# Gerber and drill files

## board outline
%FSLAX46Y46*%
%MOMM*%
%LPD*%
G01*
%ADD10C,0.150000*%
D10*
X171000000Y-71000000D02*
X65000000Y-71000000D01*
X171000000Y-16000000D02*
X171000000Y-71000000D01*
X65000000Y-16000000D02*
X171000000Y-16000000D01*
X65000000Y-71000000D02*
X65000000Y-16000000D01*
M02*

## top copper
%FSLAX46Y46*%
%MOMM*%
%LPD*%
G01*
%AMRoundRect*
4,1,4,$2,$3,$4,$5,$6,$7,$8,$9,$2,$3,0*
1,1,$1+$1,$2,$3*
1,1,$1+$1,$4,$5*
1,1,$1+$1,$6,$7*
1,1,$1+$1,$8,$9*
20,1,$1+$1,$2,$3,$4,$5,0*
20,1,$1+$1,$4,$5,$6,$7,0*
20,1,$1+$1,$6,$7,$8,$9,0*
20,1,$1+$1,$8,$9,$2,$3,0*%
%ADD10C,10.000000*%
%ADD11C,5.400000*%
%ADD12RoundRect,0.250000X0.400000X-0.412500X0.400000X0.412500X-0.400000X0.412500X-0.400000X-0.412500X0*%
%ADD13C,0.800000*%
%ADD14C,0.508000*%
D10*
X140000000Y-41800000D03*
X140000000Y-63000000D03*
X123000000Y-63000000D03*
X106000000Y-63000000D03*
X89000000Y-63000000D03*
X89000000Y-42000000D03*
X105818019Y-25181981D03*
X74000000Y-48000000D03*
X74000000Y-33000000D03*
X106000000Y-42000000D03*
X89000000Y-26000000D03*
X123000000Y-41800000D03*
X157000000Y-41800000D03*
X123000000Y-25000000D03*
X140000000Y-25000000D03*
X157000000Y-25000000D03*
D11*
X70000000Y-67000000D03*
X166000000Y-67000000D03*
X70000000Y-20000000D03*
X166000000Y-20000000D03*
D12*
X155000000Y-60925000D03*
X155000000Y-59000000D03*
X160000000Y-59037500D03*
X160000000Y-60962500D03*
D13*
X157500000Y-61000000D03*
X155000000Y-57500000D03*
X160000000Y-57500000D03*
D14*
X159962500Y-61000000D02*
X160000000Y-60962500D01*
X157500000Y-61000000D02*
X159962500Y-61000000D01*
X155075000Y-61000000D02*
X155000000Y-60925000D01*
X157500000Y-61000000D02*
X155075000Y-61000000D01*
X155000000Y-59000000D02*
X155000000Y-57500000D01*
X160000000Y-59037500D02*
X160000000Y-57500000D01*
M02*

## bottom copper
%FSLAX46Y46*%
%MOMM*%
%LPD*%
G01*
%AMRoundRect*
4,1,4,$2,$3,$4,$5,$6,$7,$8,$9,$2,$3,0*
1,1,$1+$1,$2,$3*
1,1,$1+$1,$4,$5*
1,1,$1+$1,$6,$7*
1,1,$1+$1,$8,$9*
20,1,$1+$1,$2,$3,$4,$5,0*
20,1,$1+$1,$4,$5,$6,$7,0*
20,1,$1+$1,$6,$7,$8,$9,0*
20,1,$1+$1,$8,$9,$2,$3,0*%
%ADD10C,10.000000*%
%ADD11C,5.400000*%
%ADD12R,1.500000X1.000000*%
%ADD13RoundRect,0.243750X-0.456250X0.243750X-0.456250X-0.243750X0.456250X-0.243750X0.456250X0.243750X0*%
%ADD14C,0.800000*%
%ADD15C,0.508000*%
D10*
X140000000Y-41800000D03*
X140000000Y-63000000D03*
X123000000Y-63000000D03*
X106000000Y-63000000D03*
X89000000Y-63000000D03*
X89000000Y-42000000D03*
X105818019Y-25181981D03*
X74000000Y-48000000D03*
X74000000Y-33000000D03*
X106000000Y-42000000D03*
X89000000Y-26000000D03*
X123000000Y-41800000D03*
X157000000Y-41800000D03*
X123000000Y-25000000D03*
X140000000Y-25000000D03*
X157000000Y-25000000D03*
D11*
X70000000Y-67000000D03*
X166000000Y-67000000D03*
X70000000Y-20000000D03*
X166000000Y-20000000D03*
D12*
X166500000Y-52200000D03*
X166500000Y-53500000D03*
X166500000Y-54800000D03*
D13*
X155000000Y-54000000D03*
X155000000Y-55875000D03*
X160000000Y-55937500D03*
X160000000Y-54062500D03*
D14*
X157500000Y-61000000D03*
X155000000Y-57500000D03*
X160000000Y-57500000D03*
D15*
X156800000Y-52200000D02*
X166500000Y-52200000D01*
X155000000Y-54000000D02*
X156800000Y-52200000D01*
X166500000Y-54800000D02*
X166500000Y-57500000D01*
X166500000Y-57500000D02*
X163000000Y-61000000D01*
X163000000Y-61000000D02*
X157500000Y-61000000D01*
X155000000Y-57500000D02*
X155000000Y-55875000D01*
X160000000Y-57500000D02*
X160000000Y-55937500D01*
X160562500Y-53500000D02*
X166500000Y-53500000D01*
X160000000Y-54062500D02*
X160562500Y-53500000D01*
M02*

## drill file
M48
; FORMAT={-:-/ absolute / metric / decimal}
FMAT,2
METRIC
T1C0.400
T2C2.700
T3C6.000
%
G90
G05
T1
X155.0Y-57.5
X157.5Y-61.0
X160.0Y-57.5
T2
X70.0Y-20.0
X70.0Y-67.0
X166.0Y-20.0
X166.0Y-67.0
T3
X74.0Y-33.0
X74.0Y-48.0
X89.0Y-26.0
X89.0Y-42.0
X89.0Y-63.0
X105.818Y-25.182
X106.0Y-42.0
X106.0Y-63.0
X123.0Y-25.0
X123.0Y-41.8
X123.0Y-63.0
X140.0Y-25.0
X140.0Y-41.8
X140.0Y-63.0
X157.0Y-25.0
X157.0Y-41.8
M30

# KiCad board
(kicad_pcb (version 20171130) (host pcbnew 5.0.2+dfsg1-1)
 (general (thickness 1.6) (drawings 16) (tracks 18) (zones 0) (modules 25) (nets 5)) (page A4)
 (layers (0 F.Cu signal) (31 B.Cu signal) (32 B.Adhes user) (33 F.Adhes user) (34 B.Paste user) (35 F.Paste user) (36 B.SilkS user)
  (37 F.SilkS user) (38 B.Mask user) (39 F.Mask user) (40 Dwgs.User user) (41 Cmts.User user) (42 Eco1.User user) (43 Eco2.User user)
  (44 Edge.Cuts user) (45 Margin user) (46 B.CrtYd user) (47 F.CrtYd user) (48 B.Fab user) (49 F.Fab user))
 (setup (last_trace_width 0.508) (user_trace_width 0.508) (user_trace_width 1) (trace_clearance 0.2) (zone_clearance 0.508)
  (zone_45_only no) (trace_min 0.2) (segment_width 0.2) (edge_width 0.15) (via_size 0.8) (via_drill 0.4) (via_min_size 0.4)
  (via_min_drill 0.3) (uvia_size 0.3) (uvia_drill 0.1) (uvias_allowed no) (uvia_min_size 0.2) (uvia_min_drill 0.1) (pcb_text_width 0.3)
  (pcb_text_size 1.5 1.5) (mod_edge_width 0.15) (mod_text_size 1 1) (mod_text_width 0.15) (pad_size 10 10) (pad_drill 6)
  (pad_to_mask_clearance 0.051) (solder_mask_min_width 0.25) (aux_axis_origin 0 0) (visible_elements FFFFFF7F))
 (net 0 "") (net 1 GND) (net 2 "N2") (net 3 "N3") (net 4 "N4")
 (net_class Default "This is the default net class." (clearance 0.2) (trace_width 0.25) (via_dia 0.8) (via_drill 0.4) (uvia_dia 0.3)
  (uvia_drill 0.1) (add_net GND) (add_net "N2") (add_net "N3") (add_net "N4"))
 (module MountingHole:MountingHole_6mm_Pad (layer F.Cu) (at 140 41.8)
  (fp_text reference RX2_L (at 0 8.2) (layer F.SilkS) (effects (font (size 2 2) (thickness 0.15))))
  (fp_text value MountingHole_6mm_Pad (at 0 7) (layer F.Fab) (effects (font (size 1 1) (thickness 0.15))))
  (pad 1 thru_hole circle (at 0 0) (size 10 10) (drill 6) (layers *.Cu *.Mask)))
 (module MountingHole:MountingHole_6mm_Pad (layer F.Cu) (at 140 63)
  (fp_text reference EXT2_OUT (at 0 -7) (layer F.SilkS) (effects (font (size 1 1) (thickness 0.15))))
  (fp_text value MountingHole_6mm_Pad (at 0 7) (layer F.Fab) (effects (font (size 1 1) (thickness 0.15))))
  (pad 1 thru_hole circle (at 0 0) (size 10 10) (drill 6) (layers *.Cu *.Mask)))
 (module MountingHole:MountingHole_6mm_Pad (layer F.Cu) (at 123 63)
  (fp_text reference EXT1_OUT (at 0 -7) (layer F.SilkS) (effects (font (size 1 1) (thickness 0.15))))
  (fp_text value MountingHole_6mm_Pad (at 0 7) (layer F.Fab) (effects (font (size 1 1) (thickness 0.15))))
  (pad 1 thru_hole circle (at 0 0) (size 10 10) (drill 6) (layers *.Cu *.Mask)))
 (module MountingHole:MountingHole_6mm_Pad (layer F.Cu) (at 106 63)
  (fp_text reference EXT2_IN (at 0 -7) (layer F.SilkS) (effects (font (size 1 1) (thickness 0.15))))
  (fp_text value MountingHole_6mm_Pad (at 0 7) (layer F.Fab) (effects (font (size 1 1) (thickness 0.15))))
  (pad 1 thru_hole circle (at 0 0) (size 10 10) (drill 6) (layers *.Cu *.Mask)))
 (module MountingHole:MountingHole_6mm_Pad (layer F.Cu) (at 89 63)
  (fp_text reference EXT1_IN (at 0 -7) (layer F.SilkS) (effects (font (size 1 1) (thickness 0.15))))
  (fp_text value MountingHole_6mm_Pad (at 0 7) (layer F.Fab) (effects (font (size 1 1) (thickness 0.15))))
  (pad 1 thru_hole circle (at 0 0) (size 10 10) (drill 6) (layers *.Cu *.Mask)))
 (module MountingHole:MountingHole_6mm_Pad (layer F.Cu) (at 89 42)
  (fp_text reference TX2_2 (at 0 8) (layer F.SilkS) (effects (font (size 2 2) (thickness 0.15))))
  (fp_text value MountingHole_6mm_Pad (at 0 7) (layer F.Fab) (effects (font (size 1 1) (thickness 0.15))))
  (pad 1 thru_hole circle (at 0 0) (size 10 10) (drill 6) (layers *.Cu *.Mask)))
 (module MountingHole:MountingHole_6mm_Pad (layer F.Cu) (at 105.818019 25.181981)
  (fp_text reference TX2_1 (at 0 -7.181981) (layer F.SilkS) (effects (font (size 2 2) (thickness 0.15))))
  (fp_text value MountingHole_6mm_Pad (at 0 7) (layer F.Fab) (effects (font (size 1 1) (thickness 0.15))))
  (pad 1 thru_hole circle (at 0 0) (size 10 10) (drill 6) (layers *.Cu *.Mask)))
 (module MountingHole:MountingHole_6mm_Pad (layer F.Cu) (at 74 48)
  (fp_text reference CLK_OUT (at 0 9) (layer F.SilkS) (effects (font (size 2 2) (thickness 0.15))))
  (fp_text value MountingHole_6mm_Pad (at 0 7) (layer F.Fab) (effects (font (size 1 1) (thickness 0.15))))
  (pad 1 thru_hole circle (at 0 0) (size 10 10) (drill 6) (layers *.Cu *.Mask)))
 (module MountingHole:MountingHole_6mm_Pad (layer F.Cu) (at 74 33)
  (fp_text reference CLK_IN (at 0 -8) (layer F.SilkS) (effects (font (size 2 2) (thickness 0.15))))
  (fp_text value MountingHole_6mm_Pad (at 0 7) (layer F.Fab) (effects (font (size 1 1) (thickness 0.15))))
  (pad 1 thru_hole circle (at 0 0) (size 10 10) (drill 6) (layers *.Cu *.Mask)))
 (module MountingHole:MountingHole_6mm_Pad (layer F.Cu) (at 106 42)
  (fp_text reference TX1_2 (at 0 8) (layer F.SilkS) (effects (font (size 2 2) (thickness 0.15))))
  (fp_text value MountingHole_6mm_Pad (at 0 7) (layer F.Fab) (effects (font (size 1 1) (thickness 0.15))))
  (pad 1 thru_hole circle (at 0 0) (size 10 10) (drill 6) (layers *.Cu *.Mask)))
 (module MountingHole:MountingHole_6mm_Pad (layer F.Cu) (at 89 26)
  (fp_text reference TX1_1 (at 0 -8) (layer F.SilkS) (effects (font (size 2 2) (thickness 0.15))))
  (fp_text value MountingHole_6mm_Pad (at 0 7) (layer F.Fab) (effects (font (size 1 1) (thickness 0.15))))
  (pad 1 thru_hole circle (at 0 0) (size 10 10) (drill 6) (layers *.Cu *.Mask)))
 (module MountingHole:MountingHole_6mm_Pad (layer F.Cu) (at 123 41.8)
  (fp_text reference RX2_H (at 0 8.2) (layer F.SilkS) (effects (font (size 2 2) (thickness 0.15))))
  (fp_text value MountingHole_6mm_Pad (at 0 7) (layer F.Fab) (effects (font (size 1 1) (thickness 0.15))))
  (pad 1 thru_hole circle (at 0 0) (size 10 10) (drill 6) (layers *.Cu *.Mask)))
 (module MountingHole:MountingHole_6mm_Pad (layer F.Cu) (at 157 41.8)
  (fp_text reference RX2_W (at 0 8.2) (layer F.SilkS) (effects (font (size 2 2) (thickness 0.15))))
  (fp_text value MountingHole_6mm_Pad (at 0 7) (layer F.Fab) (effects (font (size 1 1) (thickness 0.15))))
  (pad 1 thru_hole circle (at 0 0) (size 10 10) (drill 6) (layers *.Cu *.Mask)))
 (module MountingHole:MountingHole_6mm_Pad (layer F.Cu) (at 123 25)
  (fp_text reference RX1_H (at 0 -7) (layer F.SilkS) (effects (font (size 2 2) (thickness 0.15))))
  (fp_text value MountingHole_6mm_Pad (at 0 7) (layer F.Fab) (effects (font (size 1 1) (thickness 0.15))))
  (pad 1 thru_hole circle (at 0 0) (size 10 10) (drill 6) (layers *.Cu *.Mask)))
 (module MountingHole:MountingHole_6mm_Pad (layer F.Cu) (at 140 25)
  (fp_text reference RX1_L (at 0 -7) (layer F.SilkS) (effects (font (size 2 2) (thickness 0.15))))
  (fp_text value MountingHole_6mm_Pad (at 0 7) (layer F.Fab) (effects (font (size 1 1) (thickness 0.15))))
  (pad 1 thru_hole circle (at 0 0) (size 10 10) (drill 6) (layers *.Cu *.Mask)))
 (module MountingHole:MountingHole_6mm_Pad (layer F.Cu) (at 157 25)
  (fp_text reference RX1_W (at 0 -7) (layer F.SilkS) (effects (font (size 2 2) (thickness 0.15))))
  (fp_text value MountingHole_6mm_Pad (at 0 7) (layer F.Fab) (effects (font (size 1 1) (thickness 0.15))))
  (pad 1 thru_hole circle (at 0 0) (size 10 10) (drill 6) (layers *.Cu *.Mask)))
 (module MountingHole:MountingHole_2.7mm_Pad (layer F.Cu) (at 70 67)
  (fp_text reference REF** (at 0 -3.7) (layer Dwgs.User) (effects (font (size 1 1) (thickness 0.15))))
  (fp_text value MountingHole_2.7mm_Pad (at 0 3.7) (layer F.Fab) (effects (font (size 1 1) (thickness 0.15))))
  (pad 1 thru_hole circle (at 0 0) (size 5.4 5.4) (drill 2.7) (layers *.Cu *.Mask)))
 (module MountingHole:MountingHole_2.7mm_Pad (layer F.Cu) (at 166 67)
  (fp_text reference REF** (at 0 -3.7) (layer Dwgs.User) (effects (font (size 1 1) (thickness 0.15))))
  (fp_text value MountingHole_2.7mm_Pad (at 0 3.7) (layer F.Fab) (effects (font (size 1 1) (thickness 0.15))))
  (pad 1 thru_hole circle (at 0 0) (size 5.4 5.4) (drill 2.7) (layers *.Cu *.Mask)))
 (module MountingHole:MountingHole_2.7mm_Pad (layer F.Cu) (at 70 20)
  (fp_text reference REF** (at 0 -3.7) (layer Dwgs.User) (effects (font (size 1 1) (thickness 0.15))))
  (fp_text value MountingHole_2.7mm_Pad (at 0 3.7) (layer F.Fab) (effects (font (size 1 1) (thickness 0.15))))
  (pad 1 thru_hole circle (at 0 0) (size 5.4 5.4) (drill 2.7) (layers *.Cu *.Mask)))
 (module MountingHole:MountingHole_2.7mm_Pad (layer F.Cu) (at 166 20)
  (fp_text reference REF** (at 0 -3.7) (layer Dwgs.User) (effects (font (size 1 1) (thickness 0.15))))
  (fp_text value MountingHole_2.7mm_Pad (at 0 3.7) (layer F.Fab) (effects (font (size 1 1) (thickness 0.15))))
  (pad 1 thru_hole circle (at 0 0) (size 5.4 5.4) (drill 2.7) (layers *.Cu *.Mask)))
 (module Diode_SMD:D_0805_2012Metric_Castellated (layer F.Cu) (at 155 59.9625 90)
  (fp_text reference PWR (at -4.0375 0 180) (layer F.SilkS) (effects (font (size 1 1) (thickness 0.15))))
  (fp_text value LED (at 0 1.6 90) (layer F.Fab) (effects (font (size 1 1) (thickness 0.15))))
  (pad 1 smd roundrect (at -0.9625 0 90) (size 1.325 1.3) (layers F.Cu F.Paste F.Mask) (roundrect_rratio 0.192308) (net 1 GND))
  (pad 2 smd roundrect (at 0.9625 0 90) (size 1.325 1.3) (layers F.Cu F.Paste F.Mask) (roundrect_rratio 0.192308) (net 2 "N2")))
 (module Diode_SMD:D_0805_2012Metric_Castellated (layer F.Cu) (at 160 60 90)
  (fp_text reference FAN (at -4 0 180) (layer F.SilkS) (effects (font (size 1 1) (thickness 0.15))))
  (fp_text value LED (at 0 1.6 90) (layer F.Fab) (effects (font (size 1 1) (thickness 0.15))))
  (pad 2 smd roundrect (at 0.9625 0 90) (size 1.325 1.3) (layers F.Cu F.Paste F.Mask) (roundrect_rratio 0.192308) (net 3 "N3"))
  (pad 1 smd roundrect (at -0.9625 0 90) (size 1.325 1.3) (layers F.Cu F.Paste F.Mask) (roundrect_rratio 0.192308) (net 1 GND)))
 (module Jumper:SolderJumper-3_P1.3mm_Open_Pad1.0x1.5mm (layer B.Cu) (at 166.5 53.5 90)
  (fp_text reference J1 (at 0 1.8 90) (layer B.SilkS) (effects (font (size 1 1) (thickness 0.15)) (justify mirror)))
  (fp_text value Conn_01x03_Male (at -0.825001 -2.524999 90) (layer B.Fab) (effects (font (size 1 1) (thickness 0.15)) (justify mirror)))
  (pad 3 smd rect (at 1.3 0 90) (size 1 1.5) (layers B.Cu B.Mask))
  (pad 2 smd rect (at 0 0 90) (size 1 1.5) (layers B.Cu B.Mask) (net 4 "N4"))
  (pad 1 smd rect (at -1.3 0 90) (size 1 1.5) (layers B.Cu B.Mask) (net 1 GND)))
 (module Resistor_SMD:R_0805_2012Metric (layer B.Cu) (at 155 54.9375 270)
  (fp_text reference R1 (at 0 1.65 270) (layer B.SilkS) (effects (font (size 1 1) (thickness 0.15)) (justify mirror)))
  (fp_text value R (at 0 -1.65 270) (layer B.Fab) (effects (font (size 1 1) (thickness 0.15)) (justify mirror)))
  (pad 1 smd roundrect (at -0.9375 0 270) (size 0.975 1.4) (layers B.Cu B.Paste B.Mask) (roundrect_rratio 0.25))
  (pad 2 smd roundrect (at 0.9375 0 270) (size 0.975 1.4) (layers B.Cu B.Paste B.Mask) (roundrect_rratio 0.25) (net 2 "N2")))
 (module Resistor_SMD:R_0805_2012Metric (layer B.Cu) (at 160 55 270)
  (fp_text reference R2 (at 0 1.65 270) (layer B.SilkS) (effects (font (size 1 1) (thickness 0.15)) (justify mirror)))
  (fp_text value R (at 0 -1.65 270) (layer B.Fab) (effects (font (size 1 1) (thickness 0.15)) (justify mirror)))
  (pad 2 smd roundrect (at 0.9375 0 270) (size 0.975 1.4) (layers B.Cu B.Paste B.Mask) (roundrect_rratio 0.25) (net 3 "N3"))
  (pad 1 smd roundrect (at -0.9375 0 270) (size 0.975 1.4) (layers B.Cu B.Paste B.Mask) (roundrect_rratio 0.25) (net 4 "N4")))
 (gr_line (start 171 71) (end 65 71) (layer Edge.Cuts) (width 0.15))
 (gr_line (start 171 16) (end 171 71) (layer Edge.Cuts) (width 0.15))
 (gr_line (start 65 16) (end 171 16) (layer Edge.Cuts) (width 0.15))
 (gr_line (start 65 71) (end 65 16) (layer Edge.Cuts) (width 0.15))
 (segment (start 156.8 52.2) (end 166.5 52.2) (width 0.508) (layer B.Cu) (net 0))
 (segment (start 155 54) (end 156.8 52.2) (width 0.508) (layer B.Cu) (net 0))
 (segment (start 166.5 54.8) (end 166.5 57.5) (width 0.508) (layer B.Cu) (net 1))
 (via (at 157.5 61) (size 0.8) (drill 0.4) (layers F.Cu B.Cu) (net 1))
 (segment (start 166.5 57.5) (end 163 61) (width 0.508) (layer B.Cu) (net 1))
 (segment (start 163 61) (end 157.5 61) (width 0.508) (layer B.Cu) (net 1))
 (segment (start 159.9625 61) (end 160 60.9625) (width 0.508) (layer F.Cu) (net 1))
 (segment (start 157.5 61) (end 159.9625 61) (width 0.508) (layer F.Cu) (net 1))
 (segment (start 155.075 61) (end 155 60.925) (width 0.508) (layer F.Cu) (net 1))
 (segment (start 157.5 61) (end 155.075 61) (width 0.508) (layer F.Cu) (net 1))
 (via (at 155 57.5) (size 0.8) (drill 0.4) (layers F.Cu B.Cu) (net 2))
 (segment (start 155 59) (end 155 57.5) (width 0.508) (layer F.Cu) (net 2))
 (segment (start 155 57.5) (end 155 55.875) (width 0.508) (layer B.Cu) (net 2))
 (via (at 160 57.5) (size 0.8) (drill 0.4) (layers F.Cu B.Cu) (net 3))
 (segment (start 160 59.0375) (end 160 57.5) (width 0.508) (layer F.Cu) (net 3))
 (segment (start 160 57.5) (end 160 55.9375) (width 0.508) (layer B.Cu) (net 3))
 (segment (start 160.5625 53.5) (end 166.5 53.5) (width 0.508) (layer B.Cu) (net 4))
 (segment (start 160 54.0625) (end 160.5625 53.5) (width 0.508) (layer B.Cu) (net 4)))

